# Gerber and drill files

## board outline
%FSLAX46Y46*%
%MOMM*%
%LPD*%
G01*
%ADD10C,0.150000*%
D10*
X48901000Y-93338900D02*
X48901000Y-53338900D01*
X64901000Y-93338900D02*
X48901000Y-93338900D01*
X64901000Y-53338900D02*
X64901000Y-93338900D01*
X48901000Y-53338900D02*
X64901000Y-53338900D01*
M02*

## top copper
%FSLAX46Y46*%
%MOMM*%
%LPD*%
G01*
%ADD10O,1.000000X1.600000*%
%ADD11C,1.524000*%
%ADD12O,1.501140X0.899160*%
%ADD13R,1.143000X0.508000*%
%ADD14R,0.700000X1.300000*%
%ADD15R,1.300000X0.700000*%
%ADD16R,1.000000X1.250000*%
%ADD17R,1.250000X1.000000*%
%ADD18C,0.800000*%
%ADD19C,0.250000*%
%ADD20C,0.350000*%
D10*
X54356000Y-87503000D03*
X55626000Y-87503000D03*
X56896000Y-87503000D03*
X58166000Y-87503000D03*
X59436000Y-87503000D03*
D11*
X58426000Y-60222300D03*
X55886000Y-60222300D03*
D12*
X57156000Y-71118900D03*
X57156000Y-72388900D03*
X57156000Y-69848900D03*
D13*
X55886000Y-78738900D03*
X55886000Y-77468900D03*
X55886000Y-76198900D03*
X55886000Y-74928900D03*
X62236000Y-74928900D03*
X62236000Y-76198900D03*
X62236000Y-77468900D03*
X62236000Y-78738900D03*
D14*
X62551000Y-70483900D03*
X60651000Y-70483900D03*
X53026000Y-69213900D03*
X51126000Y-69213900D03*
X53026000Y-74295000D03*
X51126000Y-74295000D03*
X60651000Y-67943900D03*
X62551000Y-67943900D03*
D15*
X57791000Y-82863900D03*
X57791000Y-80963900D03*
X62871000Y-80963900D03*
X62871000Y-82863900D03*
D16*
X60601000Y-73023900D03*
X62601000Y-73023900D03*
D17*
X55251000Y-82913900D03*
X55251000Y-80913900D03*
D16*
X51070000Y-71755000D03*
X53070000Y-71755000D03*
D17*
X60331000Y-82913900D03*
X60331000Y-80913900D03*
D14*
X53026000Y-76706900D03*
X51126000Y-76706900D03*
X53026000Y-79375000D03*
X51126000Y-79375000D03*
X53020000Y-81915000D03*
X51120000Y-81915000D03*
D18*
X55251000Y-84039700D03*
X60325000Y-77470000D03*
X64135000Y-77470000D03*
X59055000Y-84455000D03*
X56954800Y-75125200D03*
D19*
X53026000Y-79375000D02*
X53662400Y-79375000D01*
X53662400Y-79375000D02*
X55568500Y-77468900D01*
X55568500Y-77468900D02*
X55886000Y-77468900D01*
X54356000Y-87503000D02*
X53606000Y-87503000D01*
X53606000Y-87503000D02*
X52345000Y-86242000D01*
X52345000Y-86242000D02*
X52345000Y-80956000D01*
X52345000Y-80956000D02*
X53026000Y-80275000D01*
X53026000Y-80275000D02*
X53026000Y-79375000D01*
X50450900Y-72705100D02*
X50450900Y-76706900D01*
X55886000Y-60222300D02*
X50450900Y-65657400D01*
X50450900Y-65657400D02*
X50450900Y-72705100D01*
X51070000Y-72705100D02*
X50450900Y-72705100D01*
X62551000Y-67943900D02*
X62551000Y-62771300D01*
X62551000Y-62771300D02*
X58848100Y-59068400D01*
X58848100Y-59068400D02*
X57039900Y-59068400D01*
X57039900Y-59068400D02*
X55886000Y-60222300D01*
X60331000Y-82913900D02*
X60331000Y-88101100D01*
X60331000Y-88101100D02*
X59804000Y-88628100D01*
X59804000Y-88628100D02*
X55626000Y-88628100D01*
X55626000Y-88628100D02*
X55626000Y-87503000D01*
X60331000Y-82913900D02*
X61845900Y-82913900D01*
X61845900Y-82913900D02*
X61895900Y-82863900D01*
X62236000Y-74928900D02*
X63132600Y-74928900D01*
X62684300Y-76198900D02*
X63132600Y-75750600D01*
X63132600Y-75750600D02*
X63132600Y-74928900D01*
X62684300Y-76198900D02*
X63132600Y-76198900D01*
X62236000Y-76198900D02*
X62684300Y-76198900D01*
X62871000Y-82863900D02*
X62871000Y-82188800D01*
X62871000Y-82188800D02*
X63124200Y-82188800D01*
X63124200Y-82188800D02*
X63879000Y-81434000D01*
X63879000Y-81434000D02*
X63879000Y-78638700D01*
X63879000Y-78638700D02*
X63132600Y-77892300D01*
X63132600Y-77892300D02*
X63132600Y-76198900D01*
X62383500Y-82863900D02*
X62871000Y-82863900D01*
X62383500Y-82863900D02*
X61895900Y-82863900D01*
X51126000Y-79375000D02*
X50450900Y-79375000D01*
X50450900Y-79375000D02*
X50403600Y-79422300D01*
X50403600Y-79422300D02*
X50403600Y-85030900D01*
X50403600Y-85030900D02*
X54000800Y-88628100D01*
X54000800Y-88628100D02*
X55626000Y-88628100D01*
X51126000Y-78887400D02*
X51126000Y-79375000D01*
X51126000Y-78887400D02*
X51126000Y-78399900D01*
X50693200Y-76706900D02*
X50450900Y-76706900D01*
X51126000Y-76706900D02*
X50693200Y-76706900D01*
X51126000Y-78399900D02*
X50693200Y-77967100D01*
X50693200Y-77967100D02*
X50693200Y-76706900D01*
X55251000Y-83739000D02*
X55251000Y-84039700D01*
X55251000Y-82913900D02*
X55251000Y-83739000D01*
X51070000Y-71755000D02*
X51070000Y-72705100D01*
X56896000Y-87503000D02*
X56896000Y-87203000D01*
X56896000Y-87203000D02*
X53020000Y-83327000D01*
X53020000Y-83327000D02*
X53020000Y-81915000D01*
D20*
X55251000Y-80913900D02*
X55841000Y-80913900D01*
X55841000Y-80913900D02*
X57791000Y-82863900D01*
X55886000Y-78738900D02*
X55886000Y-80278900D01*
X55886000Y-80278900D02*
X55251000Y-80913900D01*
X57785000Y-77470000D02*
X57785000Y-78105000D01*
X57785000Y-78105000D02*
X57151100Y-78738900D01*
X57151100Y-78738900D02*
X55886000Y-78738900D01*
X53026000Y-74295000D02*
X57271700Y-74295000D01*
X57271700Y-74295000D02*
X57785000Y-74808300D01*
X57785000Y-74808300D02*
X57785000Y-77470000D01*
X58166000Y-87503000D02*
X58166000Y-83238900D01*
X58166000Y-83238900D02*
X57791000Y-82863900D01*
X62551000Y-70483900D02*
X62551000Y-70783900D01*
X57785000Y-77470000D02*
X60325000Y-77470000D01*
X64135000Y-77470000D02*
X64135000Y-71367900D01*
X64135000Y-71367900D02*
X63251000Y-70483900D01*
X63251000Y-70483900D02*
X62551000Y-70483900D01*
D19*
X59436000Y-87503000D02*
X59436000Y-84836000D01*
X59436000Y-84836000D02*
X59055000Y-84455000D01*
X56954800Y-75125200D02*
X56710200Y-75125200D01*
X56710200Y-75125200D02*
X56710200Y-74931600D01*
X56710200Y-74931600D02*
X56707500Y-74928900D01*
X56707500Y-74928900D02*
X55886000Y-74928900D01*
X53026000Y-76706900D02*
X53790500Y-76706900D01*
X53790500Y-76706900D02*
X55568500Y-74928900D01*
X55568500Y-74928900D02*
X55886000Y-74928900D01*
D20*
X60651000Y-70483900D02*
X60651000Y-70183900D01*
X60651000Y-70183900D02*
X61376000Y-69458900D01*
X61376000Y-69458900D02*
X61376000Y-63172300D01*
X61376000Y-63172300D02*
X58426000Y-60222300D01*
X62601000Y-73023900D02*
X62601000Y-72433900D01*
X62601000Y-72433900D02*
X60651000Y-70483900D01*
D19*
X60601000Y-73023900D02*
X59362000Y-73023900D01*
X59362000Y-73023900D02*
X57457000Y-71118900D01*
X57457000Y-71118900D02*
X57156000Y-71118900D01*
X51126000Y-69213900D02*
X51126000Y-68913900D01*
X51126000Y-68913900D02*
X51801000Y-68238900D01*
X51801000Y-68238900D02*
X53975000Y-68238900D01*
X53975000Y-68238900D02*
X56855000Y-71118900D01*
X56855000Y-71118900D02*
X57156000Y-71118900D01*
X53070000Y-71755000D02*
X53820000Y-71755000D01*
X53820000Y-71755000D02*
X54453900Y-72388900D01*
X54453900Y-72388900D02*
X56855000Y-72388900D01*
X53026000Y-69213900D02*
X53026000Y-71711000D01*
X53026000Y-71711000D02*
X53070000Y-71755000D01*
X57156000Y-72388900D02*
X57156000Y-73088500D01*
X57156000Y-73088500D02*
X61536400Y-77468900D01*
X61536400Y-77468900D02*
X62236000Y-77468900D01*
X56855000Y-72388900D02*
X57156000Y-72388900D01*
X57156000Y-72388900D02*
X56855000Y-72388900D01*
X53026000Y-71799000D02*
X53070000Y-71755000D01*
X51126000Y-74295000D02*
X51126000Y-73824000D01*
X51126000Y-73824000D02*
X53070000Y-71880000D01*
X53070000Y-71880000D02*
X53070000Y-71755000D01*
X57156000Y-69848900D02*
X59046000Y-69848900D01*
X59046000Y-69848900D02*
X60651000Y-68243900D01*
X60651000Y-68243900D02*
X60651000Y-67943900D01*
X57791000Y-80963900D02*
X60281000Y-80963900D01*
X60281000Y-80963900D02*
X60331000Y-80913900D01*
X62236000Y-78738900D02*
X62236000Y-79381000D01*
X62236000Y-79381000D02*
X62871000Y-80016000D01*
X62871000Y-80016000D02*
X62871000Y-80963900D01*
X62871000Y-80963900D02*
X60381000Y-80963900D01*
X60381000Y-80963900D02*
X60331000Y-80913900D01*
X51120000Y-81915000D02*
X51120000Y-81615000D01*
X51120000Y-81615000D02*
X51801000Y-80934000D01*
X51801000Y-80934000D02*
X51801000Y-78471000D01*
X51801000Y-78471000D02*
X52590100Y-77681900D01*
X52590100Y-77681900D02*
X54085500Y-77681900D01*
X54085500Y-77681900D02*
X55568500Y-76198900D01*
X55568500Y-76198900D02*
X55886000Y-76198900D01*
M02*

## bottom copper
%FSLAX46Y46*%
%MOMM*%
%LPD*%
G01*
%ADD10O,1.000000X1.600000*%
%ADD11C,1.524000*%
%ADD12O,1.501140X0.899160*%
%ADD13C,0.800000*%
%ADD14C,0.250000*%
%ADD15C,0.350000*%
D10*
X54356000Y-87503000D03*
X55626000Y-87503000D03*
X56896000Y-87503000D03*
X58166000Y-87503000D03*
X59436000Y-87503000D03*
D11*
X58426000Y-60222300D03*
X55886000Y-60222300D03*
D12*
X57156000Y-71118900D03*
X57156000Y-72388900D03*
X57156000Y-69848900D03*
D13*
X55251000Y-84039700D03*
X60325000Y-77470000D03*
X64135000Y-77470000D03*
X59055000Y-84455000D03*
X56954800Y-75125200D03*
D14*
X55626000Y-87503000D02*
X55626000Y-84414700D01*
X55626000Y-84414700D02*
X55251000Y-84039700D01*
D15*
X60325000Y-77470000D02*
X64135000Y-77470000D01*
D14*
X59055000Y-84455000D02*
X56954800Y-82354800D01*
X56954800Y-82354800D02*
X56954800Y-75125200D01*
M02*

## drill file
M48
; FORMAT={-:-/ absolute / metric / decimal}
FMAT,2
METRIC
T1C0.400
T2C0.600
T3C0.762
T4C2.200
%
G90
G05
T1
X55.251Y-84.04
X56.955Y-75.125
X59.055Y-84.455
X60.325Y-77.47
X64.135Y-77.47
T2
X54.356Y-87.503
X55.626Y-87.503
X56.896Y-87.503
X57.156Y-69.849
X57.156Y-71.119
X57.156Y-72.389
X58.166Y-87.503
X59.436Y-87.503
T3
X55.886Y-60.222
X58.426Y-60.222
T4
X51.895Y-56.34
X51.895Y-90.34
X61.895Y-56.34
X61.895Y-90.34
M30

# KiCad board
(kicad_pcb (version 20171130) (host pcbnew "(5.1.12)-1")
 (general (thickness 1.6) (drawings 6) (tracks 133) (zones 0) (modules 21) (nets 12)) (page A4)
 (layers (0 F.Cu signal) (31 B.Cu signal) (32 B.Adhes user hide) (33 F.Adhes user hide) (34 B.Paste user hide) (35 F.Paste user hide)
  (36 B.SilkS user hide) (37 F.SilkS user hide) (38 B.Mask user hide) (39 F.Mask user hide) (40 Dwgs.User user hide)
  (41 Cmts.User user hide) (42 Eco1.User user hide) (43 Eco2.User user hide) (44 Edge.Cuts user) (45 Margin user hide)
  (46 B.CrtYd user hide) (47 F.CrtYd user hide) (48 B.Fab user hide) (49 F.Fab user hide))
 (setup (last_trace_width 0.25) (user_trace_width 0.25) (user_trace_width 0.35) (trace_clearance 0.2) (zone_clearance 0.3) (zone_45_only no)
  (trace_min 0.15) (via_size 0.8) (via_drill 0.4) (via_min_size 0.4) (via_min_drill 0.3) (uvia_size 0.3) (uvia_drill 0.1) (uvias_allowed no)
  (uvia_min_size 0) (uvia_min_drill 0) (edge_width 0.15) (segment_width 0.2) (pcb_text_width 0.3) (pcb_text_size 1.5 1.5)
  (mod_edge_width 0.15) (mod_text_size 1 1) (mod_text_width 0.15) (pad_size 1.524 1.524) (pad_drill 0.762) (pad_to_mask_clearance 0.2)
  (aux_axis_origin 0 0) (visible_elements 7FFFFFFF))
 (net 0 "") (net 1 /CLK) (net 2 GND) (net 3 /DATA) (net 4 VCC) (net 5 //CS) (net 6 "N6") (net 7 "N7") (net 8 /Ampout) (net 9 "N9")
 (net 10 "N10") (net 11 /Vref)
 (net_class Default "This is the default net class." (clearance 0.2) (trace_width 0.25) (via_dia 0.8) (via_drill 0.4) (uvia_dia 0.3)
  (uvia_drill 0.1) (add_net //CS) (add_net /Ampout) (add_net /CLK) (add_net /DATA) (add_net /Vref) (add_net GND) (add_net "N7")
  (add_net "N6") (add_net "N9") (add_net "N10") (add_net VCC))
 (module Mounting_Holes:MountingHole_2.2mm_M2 (layer F.Cu) (at 61.895 90.34)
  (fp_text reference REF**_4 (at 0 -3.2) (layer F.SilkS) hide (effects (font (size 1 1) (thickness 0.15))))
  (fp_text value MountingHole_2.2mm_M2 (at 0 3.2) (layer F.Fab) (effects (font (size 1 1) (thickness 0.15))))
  (pad 1 np_thru_hole circle (at 0 0) (size 2.2 2.2) (drill 2.2) (layers *.Cu *.Mask F.SilkS)))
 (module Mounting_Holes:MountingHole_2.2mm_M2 (layer F.Cu) (at 51.895 90.34)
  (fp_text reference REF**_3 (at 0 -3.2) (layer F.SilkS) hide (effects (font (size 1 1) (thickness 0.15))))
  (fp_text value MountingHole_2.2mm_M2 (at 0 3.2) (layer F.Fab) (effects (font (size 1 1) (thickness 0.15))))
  (pad 1 np_thru_hole circle (at 0 0) (size 2.2 2.2) (drill 2.2) (layers *.Cu *.Mask F.SilkS)))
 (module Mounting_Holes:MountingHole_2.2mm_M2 (layer F.Cu) (at 51.895 56.34)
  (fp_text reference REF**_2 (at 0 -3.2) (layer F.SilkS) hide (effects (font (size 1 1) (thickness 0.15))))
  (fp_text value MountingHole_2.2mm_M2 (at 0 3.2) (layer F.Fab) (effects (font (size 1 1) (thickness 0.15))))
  (pad 1 np_thru_hole circle (at 0 0) (size 2.2 2.2) (drill 2.2) (layers *.Cu *.Mask F.SilkS)))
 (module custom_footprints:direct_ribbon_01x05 (layer F.Cu) (at 56.896 87.503)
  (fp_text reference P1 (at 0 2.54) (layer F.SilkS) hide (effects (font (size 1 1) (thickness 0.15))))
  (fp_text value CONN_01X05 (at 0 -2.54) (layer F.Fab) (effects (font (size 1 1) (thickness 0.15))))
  (pad 1 thru_hole oval (at -2.54 0) (size 1 1.6) (drill 0.6) (layers *.Cu *.Mask F.SilkS) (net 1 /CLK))
  (pad 2 thru_hole oval (at -1.27 0) (size 1 1.6) (drill 0.6) (layers *.Cu *.Mask F.SilkS) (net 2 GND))
  (pad 3 thru_hole oval (at 0 0) (size 1 1.6) (drill 0.6) (layers *.Cu *.Mask F.SilkS) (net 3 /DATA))
  (pad 4 thru_hole oval (at 1.27 0) (size 1 1.6) (drill 0.6) (layers *.Cu *.Mask F.SilkS) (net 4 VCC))
  (pad 5 thru_hole oval (at 2.54 0) (size 1 1.6) (drill 0.6) (layers *.Cu *.Mask F.SilkS) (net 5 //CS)))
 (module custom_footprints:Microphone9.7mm (layer F.Cu) (at 57.156 62.2289 270)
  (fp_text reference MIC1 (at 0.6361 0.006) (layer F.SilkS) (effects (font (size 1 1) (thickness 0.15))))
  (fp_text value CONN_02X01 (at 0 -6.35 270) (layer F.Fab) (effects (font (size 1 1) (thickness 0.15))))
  (pad 1 thru_hole circle (at -2.0066 -1.27 270) (size 1.524 1.524) (drill 0.762) (layers *.Cu *.Mask F.SilkS) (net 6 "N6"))
  (pad 2 thru_hole circle (at -2.0066 1.27 270) (size 1.524 1.524) (drill 0.762) (layers *.Cu *.Mask F.SilkS) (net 2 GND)))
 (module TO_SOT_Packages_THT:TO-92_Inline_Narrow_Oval (layer F.Cu) (at 57.156 69.8489 270)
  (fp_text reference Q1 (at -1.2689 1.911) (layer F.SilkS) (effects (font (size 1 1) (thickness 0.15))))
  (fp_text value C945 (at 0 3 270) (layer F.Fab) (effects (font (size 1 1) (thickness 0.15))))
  (pad 2 thru_hole oval (at 1.27 0 90) (size 0.89916 1.50114) (drill 0.6) (layers *.Cu *.Mask F.SilkS) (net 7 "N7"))
  (pad 3 thru_hole oval (at 2.54 0 90) (size 0.89916 1.50114) (drill 0.6) (layers *.Cu *.Mask F.SilkS) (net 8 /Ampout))
  (pad 1 thru_hole oval (at 0 0 90) (size 0.89916 1.50114) (drill 0.6) (layers *.Cu *.Mask F.SilkS) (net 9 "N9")))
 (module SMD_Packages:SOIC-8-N (layer F.Cu) (at 59.061 76.8339 90)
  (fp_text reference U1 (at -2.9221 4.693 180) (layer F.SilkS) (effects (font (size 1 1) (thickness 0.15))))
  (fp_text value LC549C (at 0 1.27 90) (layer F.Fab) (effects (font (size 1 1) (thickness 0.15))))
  (pad 8 smd rect (at -1.905 -3.175 90) (size 0.508 1.143) (layers F.Cu F.Paste F.Mask) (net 4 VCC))
  (pad 7 smd rect (at -0.635 -3.175 90) (size 0.508 1.143) (layers F.Cu F.Paste F.Mask) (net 1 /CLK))
  (pad 6 smd rect (at 0.635 -3.175 90) (size 0.508 1.143) (layers F.Cu F.Paste F.Mask) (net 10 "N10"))
  (pad 5 smd rect (at 1.905 -3.175 90) (size 0.508 1.143) (layers F.Cu F.Paste F.Mask) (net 5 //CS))
  (pad 4 smd rect (at 1.905 3.175 90) (size 0.508 1.143) (layers F.Cu F.Paste F.Mask) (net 2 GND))
  (pad 3 smd rect (at 0.635 3.175 90) (size 0.508 1.143) (layers F.Cu F.Paste F.Mask) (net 2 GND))
  (pad 2 smd rect (at -0.635 3.175 90) (size 0.508 1.143) (layers F.Cu F.Paste F.Mask) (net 8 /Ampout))
  (pad 1 smd rect (at -1.905 3.175 90) (size 0.508 1.143) (layers F.Cu F.Paste F.Mask) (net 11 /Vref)))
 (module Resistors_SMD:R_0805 (layer F.Cu) (at 61.601 70.4839 180)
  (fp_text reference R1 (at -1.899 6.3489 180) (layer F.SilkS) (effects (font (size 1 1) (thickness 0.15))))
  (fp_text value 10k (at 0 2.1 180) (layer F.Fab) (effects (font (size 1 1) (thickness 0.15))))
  (pad 1 smd rect (at -0.95 0 180) (size 0.7 1.3) (layers F.Cu F.Paste F.Mask) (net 4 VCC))
  (pad 2 smd rect (at 0.95 0 180) (size 0.7 1.3) (layers F.Cu F.Paste F.Mask) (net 6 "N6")))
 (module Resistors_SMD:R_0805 (layer F.Cu) (at 52.076 69.2139 180)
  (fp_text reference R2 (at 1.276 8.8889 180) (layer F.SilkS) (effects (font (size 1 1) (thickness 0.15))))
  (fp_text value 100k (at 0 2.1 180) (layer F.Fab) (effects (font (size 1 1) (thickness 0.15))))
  (pad 1 smd rect (at -0.95 0 180) (size 0.7 1.3) (layers F.Cu F.Paste F.Mask) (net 8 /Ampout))
  (pad 2 smd rect (at 0.95 0 180) (size 0.7 1.3) (layers F.Cu F.Paste F.Mask) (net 7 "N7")))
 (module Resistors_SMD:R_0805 (layer F.Cu) (at 52.076 74.295 180)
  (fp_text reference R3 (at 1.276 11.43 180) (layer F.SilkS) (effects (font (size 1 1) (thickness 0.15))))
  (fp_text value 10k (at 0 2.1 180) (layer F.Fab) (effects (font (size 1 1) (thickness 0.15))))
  (pad 1 smd rect (at -0.95 0 180) (size 0.7 1.3) (layers F.Cu F.Paste F.Mask) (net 4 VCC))
  (pad 2 smd rect (at 0.95 0 180) (size 0.7 1.3) (layers F.Cu F.Paste F.Mask) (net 8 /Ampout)))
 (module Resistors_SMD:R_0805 (layer F.Cu) (at 61.601 67.9439)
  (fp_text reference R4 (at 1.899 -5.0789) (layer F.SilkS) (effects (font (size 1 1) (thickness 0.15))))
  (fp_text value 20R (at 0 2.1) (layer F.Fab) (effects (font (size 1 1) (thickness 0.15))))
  (pad 1 smd rect (at -0.95 0) (size 0.7 1.3) (layers F.Cu F.Paste F.Mask) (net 9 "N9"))
  (pad 2 smd rect (at 0.95 0) (size 0.7 1.3) (layers F.Cu F.Paste F.Mask) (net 2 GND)))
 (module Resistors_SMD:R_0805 (layer F.Cu) (at 57.791 81.9139 90)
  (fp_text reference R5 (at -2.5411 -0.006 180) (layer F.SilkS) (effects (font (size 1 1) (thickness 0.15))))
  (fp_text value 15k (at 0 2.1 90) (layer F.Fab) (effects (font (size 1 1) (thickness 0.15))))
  (pad 1 smd rect (at -0.95 0 90) (size 0.7 1.3) (layers F.Cu F.Paste F.Mask) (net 4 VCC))
  (pad 2 smd rect (at 0.95 0 90) (size 0.7 1.3) (layers F.Cu F.Paste F.Mask) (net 11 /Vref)))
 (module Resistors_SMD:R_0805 (layer F.Cu) (at 62.871 81.9139 270)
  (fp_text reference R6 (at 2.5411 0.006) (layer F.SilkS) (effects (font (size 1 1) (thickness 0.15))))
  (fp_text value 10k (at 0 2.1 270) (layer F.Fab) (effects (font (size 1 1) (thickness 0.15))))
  (pad 1 smd rect (at -0.95 0 270) (size 0.7 1.3) (layers F.Cu F.Paste F.Mask) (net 11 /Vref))
  (pad 2 smd rect (at 0.95 0 270) (size 0.7 1.3) (layers F.Cu F.Paste F.Mask) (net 2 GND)))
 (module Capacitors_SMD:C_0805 (layer F.Cu) (at 61.601 73.0239)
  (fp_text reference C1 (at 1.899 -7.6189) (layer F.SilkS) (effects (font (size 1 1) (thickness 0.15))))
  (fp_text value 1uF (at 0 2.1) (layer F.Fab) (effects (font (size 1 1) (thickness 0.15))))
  (pad 1 smd rect (at -1 0) (size 1 1.25) (layers F.Cu F.Paste F.Mask) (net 7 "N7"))
  (pad 2 smd rect (at 1 0) (size 1 1.25) (layers F.Cu F.Paste F.Mask) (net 6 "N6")))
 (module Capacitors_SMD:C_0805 (layer F.Cu) (at 55.251 81.9139 90)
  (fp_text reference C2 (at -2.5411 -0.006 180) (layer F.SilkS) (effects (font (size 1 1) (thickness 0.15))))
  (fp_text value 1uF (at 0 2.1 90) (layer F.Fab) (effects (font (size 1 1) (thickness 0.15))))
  (pad 1 smd rect (at -1 0 90) (size 1 1.25) (layers F.Cu F.Paste F.Mask) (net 2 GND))
  (pad 2 smd rect (at 1 0 90) (size 1 1.25) (layers F.Cu F.Paste F.Mask) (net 4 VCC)))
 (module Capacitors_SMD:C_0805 (layer F.Cu) (at 52.07 71.755)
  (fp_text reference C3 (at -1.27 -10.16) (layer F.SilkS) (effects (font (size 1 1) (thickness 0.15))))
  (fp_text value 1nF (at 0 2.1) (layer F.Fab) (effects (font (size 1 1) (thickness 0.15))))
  (pad 1 smd rect (at -1 0) (size 1 1.25) (layers F.Cu F.Paste F.Mask) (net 2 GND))
  (pad 2 smd rect (at 1 0) (size 1 1.25) (layers F.Cu F.Paste F.Mask) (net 8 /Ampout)))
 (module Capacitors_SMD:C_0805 (layer F.Cu) (at 60.331 81.9139 90)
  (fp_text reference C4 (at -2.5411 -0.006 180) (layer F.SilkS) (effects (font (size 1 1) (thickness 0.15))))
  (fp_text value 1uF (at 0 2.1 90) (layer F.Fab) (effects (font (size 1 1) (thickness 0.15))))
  (pad 1 smd rect (at -1 0 90) (size 1 1.25) (layers F.Cu F.Paste F.Mask) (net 2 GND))
  (pad 2 smd rect (at 1 0 90) (size 1 1.25) (layers F.Cu F.Paste F.Mask) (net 11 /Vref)))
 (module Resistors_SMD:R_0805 (layer F.Cu) (at 52.076 76.7069 180)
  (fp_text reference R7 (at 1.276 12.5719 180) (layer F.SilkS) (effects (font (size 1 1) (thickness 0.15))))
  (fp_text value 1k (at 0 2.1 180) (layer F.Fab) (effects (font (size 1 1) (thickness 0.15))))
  (pad 1 smd rect (at -0.95 0 180) (size 0.7 1.3) (layers F.Cu F.Paste F.Mask) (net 5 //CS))
  (pad 2 smd rect (at 0.95 0 180) (size 0.7 1.3) (layers F.Cu F.Paste F.Mask) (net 2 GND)))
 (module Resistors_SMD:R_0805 (layer F.Cu) (at 52.076 79.375 180)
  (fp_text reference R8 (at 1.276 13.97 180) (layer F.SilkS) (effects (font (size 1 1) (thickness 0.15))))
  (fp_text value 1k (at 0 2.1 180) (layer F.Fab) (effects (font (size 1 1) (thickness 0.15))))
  (pad 1 smd rect (at -0.95 0 180) (size 0.7 1.3) (layers F.Cu F.Paste F.Mask) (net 1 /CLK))
  (pad 2 smd rect (at 0.95 0 180) (size 0.7 1.3) (layers F.Cu F.Paste F.Mask) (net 2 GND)))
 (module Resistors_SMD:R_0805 (layer F.Cu) (at 52.07 81.915 180)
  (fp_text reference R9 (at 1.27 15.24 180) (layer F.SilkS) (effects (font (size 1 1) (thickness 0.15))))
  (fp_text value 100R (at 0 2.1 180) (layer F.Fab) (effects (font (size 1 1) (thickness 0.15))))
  (pad 1 smd rect (at -0.95 0 180) (size 0.7 1.3) (layers F.Cu F.Paste F.Mask) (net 3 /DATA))
  (pad 2 smd rect (at 0.95 0 180) (size 0.7 1.3) (layers F.Cu F.Paste F.Mask) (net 10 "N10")))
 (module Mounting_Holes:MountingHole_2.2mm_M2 (layer F.Cu) (at 61.895 56.34)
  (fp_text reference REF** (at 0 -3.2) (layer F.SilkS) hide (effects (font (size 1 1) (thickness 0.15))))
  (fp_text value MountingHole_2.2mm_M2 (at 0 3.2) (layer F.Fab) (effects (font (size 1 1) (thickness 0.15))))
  (pad 1 np_thru_hole circle (at 0 0) (size 2.2 2.2) (drill 2.2) (layers *.Cu *.Mask F.SilkS)))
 (gr_line (start 48.901 93.3389) (end 48.901 53.3389) (layer Edge.Cuts) (width 0.15))
 (gr_line (start 64.901 93.3389) (end 48.901 93.3389) (layer Edge.Cuts) (width 0.15))
 (gr_line (start 64.901 53.3389) (end 64.901 93.3389) (layer Edge.Cuts) (width 0.15))
 (gr_line (start 48.901 53.3389) (end 64.901 53.3389) (layer Edge.Cuts) (width 0.15))
 (segment (start 53.026 79.375) (end 53.6624 79.375) (width 0.25) (layer F.Cu) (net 1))
 (segment (start 53.6624 79.375) (end 55.5685 77.4689) (width 0.25) (layer F.Cu) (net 1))
 (segment (start 55.5685 77.4689) (end 55.886 77.4689) (width 0.25) (layer F.Cu) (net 1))
 (segment (start 54.356 87.503) (end 53.606 87.503) (width 0.25) (layer F.Cu) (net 1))
 (segment (start 53.606 87.503) (end 52.345 86.242) (width 0.25) (layer F.Cu) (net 1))
 (segment (start 52.345 86.242) (end 52.345 80.956) (width 0.25) (layer F.Cu) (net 1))
 (segment (start 52.345 80.956) (end 53.026 80.275) (width 0.25) (layer F.Cu) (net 1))
 (segment (start 53.026 80.275) (end 53.026 79.375) (width 0.25) (layer F.Cu) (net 1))
 (segment (start 50.4509 72.7051) (end 50.4509 76.7069) (width 0.25) (layer F.Cu) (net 2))
 (segment (start 55.886 60.2223) (end 50.4509 65.6574) (width 0.25) (layer F.Cu) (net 2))
 (segment (start 50.4509 65.6574) (end 50.4509 72.7051) (width 0.25) (layer F.Cu) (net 2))
 (segment (start 51.07 72.7051) (end 50.4509 72.7051) (width 0.25) (layer F.Cu) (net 2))
 (segment (start 62.551 67.9439) (end 62.551 62.7713) (width 0.25) (layer F.Cu) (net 2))
 (segment (start 62.551 62.7713) (end 58.8481 59.0684) (width 0.25) (layer F.Cu) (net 2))
 (segment (start 58.8481 59.0684) (end 57.0399 59.0684) (width 0.25) (layer F.Cu) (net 2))
 (segment (start 57.0399 59.0684) (end 55.886 60.2223) (width 0.25) (layer F.Cu) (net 2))
 (segment (start 60.331 82.9139) (end 60.331 88.1011) (width 0.25) (layer F.Cu) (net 2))
 (segment (start 60.331 88.1011) (end 59.804 88.6281) (width 0.25) (layer F.Cu) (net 2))
 (segment (start 59.804 88.6281) (end 55.626 88.6281) (width 0.25) (layer F.Cu) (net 2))
 (segment (start 55.626 88.6281) (end 55.626 87.503) (width 0.25) (layer F.Cu) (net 2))
 (segment (start 60.331 82.9139) (end 61.8459 82.9139) (width 0.25) (layer F.Cu) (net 2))
 (segment (start 61.8459 82.9139) (end 61.8959 82.8639) (width 0.25) (layer F.Cu) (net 2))
 (segment (start 62.236 74.9289) (end 63.1326 74.9289) (width 0.25) (layer F.Cu) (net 2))
 (segment (start 62.6843 76.1989) (end 63.1326 75.7506) (width 0.25) (layer F.Cu) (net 2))
 (segment (start 63.1326 75.7506) (end 63.1326 74.9289) (width 0.25) (layer F.Cu) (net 2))
 (segment (start 62.6843 76.1989) (end 63.1326 76.1989) (width 0.25) (layer F.Cu) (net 2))
 (segment (start 62.236 76.1989) (end 62.6843 76.1989) (width 0.25) (layer F.Cu) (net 2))
 (segment (start 62.871 82.8639) (end 62.871 82.1888) (width 0.25) (layer F.Cu) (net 2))
 (segment (start 62.871 82.1888) (end 63.1242 82.1888) (width 0.25) (layer F.Cu) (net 2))
 (segment (start 63.1242 82.1888) (end 63.879 81.434) (width 0.25) (layer F.Cu) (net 2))
 (segment (start 63.879 81.434) (end 63.879 78.6387) (width 0.25) (layer F.Cu) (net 2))
 (segment (start 63.879 78.6387) (end 63.1326 77.8923) (width 0.25) (layer F.Cu) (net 2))
 (segment (start 63.1326 77.8923) (end 63.1326 76.1989) (width 0.25) (layer F.Cu) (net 2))
 (segment (start 62.3835 82.8639) (end 62.871 82.8639) (width 0.25) (layer F.Cu) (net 2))
 (segment (start 62.3835 82.8639) (end 61.8959 82.8639) (width 0.25) (layer F.Cu) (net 2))
 (segment (start 51.126 79.375) (end 50.4509 79.375) (width 0.25) (layer F.Cu) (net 2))
 (segment (start 50.4509 79.375) (end 50.4036 79.4223) (width 0.25) (layer F.Cu) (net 2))
 (segment (start 50.4036 79.4223) (end 50.4036 85.0309) (width 0.25) (layer F.Cu) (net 2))
 (segment (start 50.4036 85.0309) (end 54.0008 88.6281) (width 0.25) (layer F.Cu) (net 2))
 (segment (start 54.0008 88.6281) (end 55.626 88.6281) (width 0.25) (layer F.Cu) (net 2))
 (segment (start 51.126 78.8874) (end 51.126 79.375) (width 0.25) (layer F.Cu) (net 2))
 (segment (start 51.126 78.8874) (end 51.126 78.3999) (width 0.25) (layer F.Cu) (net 2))
 (segment (start 50.6932 76.7069) (end 50.4509 76.7069) (width 0.25) (layer F.Cu) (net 2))
 (segment (start 51.126 76.7069) (end 50.6932 76.7069) (width 0.25) (layer F.Cu) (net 2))
 (segment (start 51.126 78.3999) (end 50.6932 77.9671) (width 0.25) (layer F.Cu) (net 2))
 (segment (start 50.6932 77.9671) (end 50.6932 76.7069) (width 0.25) (layer F.Cu) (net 2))
 (segment (start 55.251 83.739) (end 55.251 84.0397) (width 0.25) (layer F.Cu) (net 2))
 (segment (start 55.626 87.503) (end 55.626 84.4147) (width 0.25) (layer B.Cu) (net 2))
 (segment (start 55.626 84.4147) (end 55.251 84.0397) (width 0.25) (layer B.Cu) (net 2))
 (segment (start 55.251 82.9139) (end 55.251 83.739) (width 0.25) (layer F.Cu) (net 2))
 (segment (start 51.07 71.755) (end 51.07 72.7051) (width 0.25) (layer F.Cu) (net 2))
 (via (at 55.251 84.0397) (size 0.8) (layers F.Cu B.Cu) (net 2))
 (segment (start 56.896 87.503) (end 56.896 87.203) (width 0.25) (layer F.Cu) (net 3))
 (segment (start 56.896 87.203) (end 53.02 83.327) (width 0.25) (layer F.Cu) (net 3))
 (segment (start 53.02 83.327) (end 53.02 81.915) (width 0.25) (layer F.Cu) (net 3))
 (segment (start 55.251 80.9139) (end 55.841 80.9139) (width 0.35) (layer F.Cu) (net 4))
 (segment (start 55.841 80.9139) (end 57.791 82.8639) (width 0.35) (layer F.Cu) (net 4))
 (segment (start 55.886 78.7389) (end 55.886 80.2789) (width 0.35) (layer F.Cu) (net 4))
 (segment (start 55.886 80.2789) (end 55.251 80.9139) (width 0.35) (layer F.Cu) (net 4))
 (segment (start 57.785 77.47) (end 57.785 78.105) (width 0.35) (layer F.Cu) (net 4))
 (segment (start 57.785 78.105) (end 57.1511 78.7389) (width 0.35) (layer F.Cu) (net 4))
 (segment (start 57.1511 78.7389) (end 55.886 78.7389) (width 0.35) (layer F.Cu) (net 4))
 (segment (start 53.026 74.295) (end 57.2717 74.295) (width 0.35) (layer F.Cu) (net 4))
 (segment (start 57.2717 74.295) (end 57.785 74.8083) (width 0.35) (layer F.Cu) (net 4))
 (segment (start 57.785 74.8083) (end 57.785 77.47) (width 0.35) (layer F.Cu) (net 4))
 (segment (start 58.166 87.503) (end 58.166 83.2389) (width 0.35) (layer F.Cu) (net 4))
 (segment (start 58.166 83.2389) (end 57.791 82.8639) (width 0.35) (layer F.Cu) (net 4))
 (segment (start 62.551 70.4839) (end 62.551 70.7839) (width 0.35) (layer F.Cu) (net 4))
 (segment (start 57.785 77.47) (end 60.325 77.47) (width 0.35) (layer F.Cu) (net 4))
 (segment (start 60.325 77.47) (end 64.135 77.47) (width 0.35) (layer B.Cu) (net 4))
 (segment (start 64.135 77.47) (end 64.135 71.3679) (width 0.35) (layer F.Cu) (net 4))
 (segment (start 64.135 71.3679) (end 63.251 70.4839) (width 0.35) (layer F.Cu) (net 4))
 (segment (start 63.251 70.4839) (end 62.551 70.4839) (width 0.35) (layer F.Cu) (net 4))
 (via (at 60.325 77.47) (size 0.8) (layers F.Cu B.Cu) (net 4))
 (via (at 64.135 77.47) (size 0.8) (layers F.Cu B.Cu) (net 4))
 (segment (start 59.436 87.503) (end 59.436 84.836) (width 0.25) (layer F.Cu) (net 5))
 (segment (start 59.436 84.836) (end 59.055 84.455) (width 0.25) (layer F.Cu) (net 5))
 (segment (start 59.055 84.455) (end 56.9548 82.3548) (width 0.25) (layer B.Cu) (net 5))
 (segment (start 56.9548 82.3548) (end 56.9548 75.1252) (width 0.25) (layer B.Cu) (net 5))
 (segment (start 56.9548 75.1252) (end 56.7102 75.1252) (width 0.25) (layer F.Cu) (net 5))
 (segment (start 56.7102 75.1252) (end 56.7102 74.9316) (width 0.25) (layer F.Cu) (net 5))
 (segment (start 56.7102 74.9316) (end 56.7075 74.9289) (width 0.25) (layer F.Cu) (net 5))
 (segment (start 56.7075 74.9289) (end 55.886 74.9289) (width 0.25) (layer F.Cu) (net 5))
 (segment (start 53.026 76.7069) (end 53.7905 76.7069) (width 0.25) (layer F.Cu) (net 5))
 (segment (start 53.7905 76.7069) (end 55.5685 74.9289) (width 0.25) (layer F.Cu) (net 5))
 (segment (start 55.5685 74.9289) (end 55.886 74.9289) (width 0.25) (layer F.Cu) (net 5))
 (via (at 59.055 84.455) (size 0.8) (layers F.Cu B.Cu) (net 5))
 (via (at 56.9548 75.1252) (size 0.8) (layers F.Cu B.Cu) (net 5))
 (segment (start 60.651 70.4839) (end 60.651 70.1839) (width 0.35) (layer F.Cu) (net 6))
 (segment (start 60.651 70.1839) (end 61.376 69.4589) (width 0.35) (layer F.Cu) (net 6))
 (segment (start 61.376 69.4589) (end 61.376 63.1723) (width 0.35) (layer F.Cu) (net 6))
 (segment (start 61.376 63.1723) (end 58.426 60.2223) (width 0.35) (layer F.Cu) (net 6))
 (segment (start 62.601 73.0239) (end 62.601 72.4339) (width 0.35) (layer F.Cu) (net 6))
 (segment (start 62.601 72.4339) (end 60.651 70.4839) (width 0.35) (layer F.Cu) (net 6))
 (segment (start 60.601 73.0239) (end 59.362 73.0239) (width 0.25) (layer F.Cu) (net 7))
 (segment (start 59.362 73.0239) (end 57.457 71.1189) (width 0.25) (layer F.Cu) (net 7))
 (segment (start 57.457 71.1189) (end 57.156 71.1189) (width 0.25) (layer F.Cu) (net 7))
 (segment (start 51.126 69.2139) (end 51.126 68.9139) (width 0.25) (layer F.Cu) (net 7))
 (segment (start 51.126 68.9139) (end 51.801 68.2389) (width 0.25) (layer F.Cu) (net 7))
 (segment (start 51.801 68.2389) (end 53.975 68.2389) (width 0.25) (layer F.Cu) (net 7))
 (segment (start 53.975 68.2389) (end 56.855 71.1189) (width 0.25) (layer F.Cu) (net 7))
 (segment (start 56.855 71.1189) (end 57.156 71.1189) (width 0.25) (layer F.Cu) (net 7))
 (segment (start 53.07 71.755) (end 53.82 71.755) (width 0.25) (layer F.Cu) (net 8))
 (segment (start 53.82 71.755) (end 54.4539 72.3889) (width 0.25) (layer F.Cu) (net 8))
 (segment (start 54.4539 72.3889) (end 56.855 72.3889) (width 0.25) (layer F.Cu) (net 8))
 (segment (start 53.026 69.2139) (end 53.026 71.711) (width 0.25) (layer F.Cu) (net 8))
 (segment (start 53.026 71.711) (end 53.07 71.755) (width 0.25) (layer F.Cu) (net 8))
 (segment (start 57.156 72.3889) (end 57.156 73.0885) (width 0.25) (layer F.Cu) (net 8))
 (segment (start 57.156 73.0885) (end 61.5364 77.4689) (width 0.25) (layer F.Cu) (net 8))
 (segment (start 61.5364 77.4689) (end 62.236 77.4689) (width 0.25) (layer F.Cu) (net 8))
 (segment (start 56.855 72.3889) (end 57.156 72.3889) (width 0.25) (layer F.Cu) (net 8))
 (segment (start 57.156 72.3889) (end 56.855 72.3889) (width 0.25) (layer F.Cu) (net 8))
 (segment (start 53.026 71.799) (end 53.07 71.755) (width 0.25) (layer F.Cu) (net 8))
 (segment (start 51.126 74.295) (end 51.126 73.824) (width 0.25) (layer F.Cu) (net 8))
 (segment (start 51.126 73.824) (end 53.07 71.88) (width 0.25) (layer F.Cu) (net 8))
 (segment (start 53.07 71.88) (end 53.07 71.755) (width 0.25) (layer F.Cu) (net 8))
 (segment (start 57.156 69.8489) (end 59.046 69.8489) (width 0.25) (layer F.Cu) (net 9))
 (segment (start 59.046 69.8489) (end 60.651 68.2439) (width 0.25) (layer F.Cu) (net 9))
 (segment (start 60.651 68.2439) (end 60.651 67.9439) (width 0.25) (layer F.Cu) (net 9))
 (segment (start 57.791 80.9639) (end 60.281 80.9639) (width 0.25) (layer F.Cu) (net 11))
 (segment (start 60.281 80.9639) (end 60.331 80.9139) (width 0.25) (layer F.Cu) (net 11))
 (segment (start 62.236 78.7389) (end 62.236 79.381) (width 0.25) (layer F.Cu) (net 11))
 (segment (start 62.236 79.381) (end 62.871 80.016) (width 0.25) (layer F.Cu) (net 11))
 (segment (start 62.871 80.016) (end 62.871 80.9639) (width 0.25) (layer F.Cu) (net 11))
 (segment (start 62.871 80.9639) (end 60.381 80.9639) (width 0.25) (layer F.Cu) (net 11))
 (segment (start 60.381 80.9639) (end 60.331 80.9139) (width 0.25) (layer F.Cu) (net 11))
 (segment (start 51.12 81.915) (end 51.12 81.615) (width 0.25) (layer F.Cu) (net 10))
 (segment (start 51.12 81.615) (end 51.801 80.934) (width 0.25) (layer F.Cu) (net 10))
 (segment (start 51.801 80.934) (end 51.801 78.471) (width 0.25) (layer F.Cu) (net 10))
 (segment (start 51.801 78.471) (end 52.5901 77.6819) (width 0.25) (layer F.Cu) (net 10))
 (segment (start 52.5901 77.6819) (end 54.0855 77.6819) (width 0.25) (layer F.Cu) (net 10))
 (segment (start 54.0855 77.6819) (end 55.5685 76.1989) (width 0.25) (layer F.Cu) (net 10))
 (segment (start 55.5685 76.1989) (end 55.886 76.1989) (width 0.25) (layer F.Cu) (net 10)))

